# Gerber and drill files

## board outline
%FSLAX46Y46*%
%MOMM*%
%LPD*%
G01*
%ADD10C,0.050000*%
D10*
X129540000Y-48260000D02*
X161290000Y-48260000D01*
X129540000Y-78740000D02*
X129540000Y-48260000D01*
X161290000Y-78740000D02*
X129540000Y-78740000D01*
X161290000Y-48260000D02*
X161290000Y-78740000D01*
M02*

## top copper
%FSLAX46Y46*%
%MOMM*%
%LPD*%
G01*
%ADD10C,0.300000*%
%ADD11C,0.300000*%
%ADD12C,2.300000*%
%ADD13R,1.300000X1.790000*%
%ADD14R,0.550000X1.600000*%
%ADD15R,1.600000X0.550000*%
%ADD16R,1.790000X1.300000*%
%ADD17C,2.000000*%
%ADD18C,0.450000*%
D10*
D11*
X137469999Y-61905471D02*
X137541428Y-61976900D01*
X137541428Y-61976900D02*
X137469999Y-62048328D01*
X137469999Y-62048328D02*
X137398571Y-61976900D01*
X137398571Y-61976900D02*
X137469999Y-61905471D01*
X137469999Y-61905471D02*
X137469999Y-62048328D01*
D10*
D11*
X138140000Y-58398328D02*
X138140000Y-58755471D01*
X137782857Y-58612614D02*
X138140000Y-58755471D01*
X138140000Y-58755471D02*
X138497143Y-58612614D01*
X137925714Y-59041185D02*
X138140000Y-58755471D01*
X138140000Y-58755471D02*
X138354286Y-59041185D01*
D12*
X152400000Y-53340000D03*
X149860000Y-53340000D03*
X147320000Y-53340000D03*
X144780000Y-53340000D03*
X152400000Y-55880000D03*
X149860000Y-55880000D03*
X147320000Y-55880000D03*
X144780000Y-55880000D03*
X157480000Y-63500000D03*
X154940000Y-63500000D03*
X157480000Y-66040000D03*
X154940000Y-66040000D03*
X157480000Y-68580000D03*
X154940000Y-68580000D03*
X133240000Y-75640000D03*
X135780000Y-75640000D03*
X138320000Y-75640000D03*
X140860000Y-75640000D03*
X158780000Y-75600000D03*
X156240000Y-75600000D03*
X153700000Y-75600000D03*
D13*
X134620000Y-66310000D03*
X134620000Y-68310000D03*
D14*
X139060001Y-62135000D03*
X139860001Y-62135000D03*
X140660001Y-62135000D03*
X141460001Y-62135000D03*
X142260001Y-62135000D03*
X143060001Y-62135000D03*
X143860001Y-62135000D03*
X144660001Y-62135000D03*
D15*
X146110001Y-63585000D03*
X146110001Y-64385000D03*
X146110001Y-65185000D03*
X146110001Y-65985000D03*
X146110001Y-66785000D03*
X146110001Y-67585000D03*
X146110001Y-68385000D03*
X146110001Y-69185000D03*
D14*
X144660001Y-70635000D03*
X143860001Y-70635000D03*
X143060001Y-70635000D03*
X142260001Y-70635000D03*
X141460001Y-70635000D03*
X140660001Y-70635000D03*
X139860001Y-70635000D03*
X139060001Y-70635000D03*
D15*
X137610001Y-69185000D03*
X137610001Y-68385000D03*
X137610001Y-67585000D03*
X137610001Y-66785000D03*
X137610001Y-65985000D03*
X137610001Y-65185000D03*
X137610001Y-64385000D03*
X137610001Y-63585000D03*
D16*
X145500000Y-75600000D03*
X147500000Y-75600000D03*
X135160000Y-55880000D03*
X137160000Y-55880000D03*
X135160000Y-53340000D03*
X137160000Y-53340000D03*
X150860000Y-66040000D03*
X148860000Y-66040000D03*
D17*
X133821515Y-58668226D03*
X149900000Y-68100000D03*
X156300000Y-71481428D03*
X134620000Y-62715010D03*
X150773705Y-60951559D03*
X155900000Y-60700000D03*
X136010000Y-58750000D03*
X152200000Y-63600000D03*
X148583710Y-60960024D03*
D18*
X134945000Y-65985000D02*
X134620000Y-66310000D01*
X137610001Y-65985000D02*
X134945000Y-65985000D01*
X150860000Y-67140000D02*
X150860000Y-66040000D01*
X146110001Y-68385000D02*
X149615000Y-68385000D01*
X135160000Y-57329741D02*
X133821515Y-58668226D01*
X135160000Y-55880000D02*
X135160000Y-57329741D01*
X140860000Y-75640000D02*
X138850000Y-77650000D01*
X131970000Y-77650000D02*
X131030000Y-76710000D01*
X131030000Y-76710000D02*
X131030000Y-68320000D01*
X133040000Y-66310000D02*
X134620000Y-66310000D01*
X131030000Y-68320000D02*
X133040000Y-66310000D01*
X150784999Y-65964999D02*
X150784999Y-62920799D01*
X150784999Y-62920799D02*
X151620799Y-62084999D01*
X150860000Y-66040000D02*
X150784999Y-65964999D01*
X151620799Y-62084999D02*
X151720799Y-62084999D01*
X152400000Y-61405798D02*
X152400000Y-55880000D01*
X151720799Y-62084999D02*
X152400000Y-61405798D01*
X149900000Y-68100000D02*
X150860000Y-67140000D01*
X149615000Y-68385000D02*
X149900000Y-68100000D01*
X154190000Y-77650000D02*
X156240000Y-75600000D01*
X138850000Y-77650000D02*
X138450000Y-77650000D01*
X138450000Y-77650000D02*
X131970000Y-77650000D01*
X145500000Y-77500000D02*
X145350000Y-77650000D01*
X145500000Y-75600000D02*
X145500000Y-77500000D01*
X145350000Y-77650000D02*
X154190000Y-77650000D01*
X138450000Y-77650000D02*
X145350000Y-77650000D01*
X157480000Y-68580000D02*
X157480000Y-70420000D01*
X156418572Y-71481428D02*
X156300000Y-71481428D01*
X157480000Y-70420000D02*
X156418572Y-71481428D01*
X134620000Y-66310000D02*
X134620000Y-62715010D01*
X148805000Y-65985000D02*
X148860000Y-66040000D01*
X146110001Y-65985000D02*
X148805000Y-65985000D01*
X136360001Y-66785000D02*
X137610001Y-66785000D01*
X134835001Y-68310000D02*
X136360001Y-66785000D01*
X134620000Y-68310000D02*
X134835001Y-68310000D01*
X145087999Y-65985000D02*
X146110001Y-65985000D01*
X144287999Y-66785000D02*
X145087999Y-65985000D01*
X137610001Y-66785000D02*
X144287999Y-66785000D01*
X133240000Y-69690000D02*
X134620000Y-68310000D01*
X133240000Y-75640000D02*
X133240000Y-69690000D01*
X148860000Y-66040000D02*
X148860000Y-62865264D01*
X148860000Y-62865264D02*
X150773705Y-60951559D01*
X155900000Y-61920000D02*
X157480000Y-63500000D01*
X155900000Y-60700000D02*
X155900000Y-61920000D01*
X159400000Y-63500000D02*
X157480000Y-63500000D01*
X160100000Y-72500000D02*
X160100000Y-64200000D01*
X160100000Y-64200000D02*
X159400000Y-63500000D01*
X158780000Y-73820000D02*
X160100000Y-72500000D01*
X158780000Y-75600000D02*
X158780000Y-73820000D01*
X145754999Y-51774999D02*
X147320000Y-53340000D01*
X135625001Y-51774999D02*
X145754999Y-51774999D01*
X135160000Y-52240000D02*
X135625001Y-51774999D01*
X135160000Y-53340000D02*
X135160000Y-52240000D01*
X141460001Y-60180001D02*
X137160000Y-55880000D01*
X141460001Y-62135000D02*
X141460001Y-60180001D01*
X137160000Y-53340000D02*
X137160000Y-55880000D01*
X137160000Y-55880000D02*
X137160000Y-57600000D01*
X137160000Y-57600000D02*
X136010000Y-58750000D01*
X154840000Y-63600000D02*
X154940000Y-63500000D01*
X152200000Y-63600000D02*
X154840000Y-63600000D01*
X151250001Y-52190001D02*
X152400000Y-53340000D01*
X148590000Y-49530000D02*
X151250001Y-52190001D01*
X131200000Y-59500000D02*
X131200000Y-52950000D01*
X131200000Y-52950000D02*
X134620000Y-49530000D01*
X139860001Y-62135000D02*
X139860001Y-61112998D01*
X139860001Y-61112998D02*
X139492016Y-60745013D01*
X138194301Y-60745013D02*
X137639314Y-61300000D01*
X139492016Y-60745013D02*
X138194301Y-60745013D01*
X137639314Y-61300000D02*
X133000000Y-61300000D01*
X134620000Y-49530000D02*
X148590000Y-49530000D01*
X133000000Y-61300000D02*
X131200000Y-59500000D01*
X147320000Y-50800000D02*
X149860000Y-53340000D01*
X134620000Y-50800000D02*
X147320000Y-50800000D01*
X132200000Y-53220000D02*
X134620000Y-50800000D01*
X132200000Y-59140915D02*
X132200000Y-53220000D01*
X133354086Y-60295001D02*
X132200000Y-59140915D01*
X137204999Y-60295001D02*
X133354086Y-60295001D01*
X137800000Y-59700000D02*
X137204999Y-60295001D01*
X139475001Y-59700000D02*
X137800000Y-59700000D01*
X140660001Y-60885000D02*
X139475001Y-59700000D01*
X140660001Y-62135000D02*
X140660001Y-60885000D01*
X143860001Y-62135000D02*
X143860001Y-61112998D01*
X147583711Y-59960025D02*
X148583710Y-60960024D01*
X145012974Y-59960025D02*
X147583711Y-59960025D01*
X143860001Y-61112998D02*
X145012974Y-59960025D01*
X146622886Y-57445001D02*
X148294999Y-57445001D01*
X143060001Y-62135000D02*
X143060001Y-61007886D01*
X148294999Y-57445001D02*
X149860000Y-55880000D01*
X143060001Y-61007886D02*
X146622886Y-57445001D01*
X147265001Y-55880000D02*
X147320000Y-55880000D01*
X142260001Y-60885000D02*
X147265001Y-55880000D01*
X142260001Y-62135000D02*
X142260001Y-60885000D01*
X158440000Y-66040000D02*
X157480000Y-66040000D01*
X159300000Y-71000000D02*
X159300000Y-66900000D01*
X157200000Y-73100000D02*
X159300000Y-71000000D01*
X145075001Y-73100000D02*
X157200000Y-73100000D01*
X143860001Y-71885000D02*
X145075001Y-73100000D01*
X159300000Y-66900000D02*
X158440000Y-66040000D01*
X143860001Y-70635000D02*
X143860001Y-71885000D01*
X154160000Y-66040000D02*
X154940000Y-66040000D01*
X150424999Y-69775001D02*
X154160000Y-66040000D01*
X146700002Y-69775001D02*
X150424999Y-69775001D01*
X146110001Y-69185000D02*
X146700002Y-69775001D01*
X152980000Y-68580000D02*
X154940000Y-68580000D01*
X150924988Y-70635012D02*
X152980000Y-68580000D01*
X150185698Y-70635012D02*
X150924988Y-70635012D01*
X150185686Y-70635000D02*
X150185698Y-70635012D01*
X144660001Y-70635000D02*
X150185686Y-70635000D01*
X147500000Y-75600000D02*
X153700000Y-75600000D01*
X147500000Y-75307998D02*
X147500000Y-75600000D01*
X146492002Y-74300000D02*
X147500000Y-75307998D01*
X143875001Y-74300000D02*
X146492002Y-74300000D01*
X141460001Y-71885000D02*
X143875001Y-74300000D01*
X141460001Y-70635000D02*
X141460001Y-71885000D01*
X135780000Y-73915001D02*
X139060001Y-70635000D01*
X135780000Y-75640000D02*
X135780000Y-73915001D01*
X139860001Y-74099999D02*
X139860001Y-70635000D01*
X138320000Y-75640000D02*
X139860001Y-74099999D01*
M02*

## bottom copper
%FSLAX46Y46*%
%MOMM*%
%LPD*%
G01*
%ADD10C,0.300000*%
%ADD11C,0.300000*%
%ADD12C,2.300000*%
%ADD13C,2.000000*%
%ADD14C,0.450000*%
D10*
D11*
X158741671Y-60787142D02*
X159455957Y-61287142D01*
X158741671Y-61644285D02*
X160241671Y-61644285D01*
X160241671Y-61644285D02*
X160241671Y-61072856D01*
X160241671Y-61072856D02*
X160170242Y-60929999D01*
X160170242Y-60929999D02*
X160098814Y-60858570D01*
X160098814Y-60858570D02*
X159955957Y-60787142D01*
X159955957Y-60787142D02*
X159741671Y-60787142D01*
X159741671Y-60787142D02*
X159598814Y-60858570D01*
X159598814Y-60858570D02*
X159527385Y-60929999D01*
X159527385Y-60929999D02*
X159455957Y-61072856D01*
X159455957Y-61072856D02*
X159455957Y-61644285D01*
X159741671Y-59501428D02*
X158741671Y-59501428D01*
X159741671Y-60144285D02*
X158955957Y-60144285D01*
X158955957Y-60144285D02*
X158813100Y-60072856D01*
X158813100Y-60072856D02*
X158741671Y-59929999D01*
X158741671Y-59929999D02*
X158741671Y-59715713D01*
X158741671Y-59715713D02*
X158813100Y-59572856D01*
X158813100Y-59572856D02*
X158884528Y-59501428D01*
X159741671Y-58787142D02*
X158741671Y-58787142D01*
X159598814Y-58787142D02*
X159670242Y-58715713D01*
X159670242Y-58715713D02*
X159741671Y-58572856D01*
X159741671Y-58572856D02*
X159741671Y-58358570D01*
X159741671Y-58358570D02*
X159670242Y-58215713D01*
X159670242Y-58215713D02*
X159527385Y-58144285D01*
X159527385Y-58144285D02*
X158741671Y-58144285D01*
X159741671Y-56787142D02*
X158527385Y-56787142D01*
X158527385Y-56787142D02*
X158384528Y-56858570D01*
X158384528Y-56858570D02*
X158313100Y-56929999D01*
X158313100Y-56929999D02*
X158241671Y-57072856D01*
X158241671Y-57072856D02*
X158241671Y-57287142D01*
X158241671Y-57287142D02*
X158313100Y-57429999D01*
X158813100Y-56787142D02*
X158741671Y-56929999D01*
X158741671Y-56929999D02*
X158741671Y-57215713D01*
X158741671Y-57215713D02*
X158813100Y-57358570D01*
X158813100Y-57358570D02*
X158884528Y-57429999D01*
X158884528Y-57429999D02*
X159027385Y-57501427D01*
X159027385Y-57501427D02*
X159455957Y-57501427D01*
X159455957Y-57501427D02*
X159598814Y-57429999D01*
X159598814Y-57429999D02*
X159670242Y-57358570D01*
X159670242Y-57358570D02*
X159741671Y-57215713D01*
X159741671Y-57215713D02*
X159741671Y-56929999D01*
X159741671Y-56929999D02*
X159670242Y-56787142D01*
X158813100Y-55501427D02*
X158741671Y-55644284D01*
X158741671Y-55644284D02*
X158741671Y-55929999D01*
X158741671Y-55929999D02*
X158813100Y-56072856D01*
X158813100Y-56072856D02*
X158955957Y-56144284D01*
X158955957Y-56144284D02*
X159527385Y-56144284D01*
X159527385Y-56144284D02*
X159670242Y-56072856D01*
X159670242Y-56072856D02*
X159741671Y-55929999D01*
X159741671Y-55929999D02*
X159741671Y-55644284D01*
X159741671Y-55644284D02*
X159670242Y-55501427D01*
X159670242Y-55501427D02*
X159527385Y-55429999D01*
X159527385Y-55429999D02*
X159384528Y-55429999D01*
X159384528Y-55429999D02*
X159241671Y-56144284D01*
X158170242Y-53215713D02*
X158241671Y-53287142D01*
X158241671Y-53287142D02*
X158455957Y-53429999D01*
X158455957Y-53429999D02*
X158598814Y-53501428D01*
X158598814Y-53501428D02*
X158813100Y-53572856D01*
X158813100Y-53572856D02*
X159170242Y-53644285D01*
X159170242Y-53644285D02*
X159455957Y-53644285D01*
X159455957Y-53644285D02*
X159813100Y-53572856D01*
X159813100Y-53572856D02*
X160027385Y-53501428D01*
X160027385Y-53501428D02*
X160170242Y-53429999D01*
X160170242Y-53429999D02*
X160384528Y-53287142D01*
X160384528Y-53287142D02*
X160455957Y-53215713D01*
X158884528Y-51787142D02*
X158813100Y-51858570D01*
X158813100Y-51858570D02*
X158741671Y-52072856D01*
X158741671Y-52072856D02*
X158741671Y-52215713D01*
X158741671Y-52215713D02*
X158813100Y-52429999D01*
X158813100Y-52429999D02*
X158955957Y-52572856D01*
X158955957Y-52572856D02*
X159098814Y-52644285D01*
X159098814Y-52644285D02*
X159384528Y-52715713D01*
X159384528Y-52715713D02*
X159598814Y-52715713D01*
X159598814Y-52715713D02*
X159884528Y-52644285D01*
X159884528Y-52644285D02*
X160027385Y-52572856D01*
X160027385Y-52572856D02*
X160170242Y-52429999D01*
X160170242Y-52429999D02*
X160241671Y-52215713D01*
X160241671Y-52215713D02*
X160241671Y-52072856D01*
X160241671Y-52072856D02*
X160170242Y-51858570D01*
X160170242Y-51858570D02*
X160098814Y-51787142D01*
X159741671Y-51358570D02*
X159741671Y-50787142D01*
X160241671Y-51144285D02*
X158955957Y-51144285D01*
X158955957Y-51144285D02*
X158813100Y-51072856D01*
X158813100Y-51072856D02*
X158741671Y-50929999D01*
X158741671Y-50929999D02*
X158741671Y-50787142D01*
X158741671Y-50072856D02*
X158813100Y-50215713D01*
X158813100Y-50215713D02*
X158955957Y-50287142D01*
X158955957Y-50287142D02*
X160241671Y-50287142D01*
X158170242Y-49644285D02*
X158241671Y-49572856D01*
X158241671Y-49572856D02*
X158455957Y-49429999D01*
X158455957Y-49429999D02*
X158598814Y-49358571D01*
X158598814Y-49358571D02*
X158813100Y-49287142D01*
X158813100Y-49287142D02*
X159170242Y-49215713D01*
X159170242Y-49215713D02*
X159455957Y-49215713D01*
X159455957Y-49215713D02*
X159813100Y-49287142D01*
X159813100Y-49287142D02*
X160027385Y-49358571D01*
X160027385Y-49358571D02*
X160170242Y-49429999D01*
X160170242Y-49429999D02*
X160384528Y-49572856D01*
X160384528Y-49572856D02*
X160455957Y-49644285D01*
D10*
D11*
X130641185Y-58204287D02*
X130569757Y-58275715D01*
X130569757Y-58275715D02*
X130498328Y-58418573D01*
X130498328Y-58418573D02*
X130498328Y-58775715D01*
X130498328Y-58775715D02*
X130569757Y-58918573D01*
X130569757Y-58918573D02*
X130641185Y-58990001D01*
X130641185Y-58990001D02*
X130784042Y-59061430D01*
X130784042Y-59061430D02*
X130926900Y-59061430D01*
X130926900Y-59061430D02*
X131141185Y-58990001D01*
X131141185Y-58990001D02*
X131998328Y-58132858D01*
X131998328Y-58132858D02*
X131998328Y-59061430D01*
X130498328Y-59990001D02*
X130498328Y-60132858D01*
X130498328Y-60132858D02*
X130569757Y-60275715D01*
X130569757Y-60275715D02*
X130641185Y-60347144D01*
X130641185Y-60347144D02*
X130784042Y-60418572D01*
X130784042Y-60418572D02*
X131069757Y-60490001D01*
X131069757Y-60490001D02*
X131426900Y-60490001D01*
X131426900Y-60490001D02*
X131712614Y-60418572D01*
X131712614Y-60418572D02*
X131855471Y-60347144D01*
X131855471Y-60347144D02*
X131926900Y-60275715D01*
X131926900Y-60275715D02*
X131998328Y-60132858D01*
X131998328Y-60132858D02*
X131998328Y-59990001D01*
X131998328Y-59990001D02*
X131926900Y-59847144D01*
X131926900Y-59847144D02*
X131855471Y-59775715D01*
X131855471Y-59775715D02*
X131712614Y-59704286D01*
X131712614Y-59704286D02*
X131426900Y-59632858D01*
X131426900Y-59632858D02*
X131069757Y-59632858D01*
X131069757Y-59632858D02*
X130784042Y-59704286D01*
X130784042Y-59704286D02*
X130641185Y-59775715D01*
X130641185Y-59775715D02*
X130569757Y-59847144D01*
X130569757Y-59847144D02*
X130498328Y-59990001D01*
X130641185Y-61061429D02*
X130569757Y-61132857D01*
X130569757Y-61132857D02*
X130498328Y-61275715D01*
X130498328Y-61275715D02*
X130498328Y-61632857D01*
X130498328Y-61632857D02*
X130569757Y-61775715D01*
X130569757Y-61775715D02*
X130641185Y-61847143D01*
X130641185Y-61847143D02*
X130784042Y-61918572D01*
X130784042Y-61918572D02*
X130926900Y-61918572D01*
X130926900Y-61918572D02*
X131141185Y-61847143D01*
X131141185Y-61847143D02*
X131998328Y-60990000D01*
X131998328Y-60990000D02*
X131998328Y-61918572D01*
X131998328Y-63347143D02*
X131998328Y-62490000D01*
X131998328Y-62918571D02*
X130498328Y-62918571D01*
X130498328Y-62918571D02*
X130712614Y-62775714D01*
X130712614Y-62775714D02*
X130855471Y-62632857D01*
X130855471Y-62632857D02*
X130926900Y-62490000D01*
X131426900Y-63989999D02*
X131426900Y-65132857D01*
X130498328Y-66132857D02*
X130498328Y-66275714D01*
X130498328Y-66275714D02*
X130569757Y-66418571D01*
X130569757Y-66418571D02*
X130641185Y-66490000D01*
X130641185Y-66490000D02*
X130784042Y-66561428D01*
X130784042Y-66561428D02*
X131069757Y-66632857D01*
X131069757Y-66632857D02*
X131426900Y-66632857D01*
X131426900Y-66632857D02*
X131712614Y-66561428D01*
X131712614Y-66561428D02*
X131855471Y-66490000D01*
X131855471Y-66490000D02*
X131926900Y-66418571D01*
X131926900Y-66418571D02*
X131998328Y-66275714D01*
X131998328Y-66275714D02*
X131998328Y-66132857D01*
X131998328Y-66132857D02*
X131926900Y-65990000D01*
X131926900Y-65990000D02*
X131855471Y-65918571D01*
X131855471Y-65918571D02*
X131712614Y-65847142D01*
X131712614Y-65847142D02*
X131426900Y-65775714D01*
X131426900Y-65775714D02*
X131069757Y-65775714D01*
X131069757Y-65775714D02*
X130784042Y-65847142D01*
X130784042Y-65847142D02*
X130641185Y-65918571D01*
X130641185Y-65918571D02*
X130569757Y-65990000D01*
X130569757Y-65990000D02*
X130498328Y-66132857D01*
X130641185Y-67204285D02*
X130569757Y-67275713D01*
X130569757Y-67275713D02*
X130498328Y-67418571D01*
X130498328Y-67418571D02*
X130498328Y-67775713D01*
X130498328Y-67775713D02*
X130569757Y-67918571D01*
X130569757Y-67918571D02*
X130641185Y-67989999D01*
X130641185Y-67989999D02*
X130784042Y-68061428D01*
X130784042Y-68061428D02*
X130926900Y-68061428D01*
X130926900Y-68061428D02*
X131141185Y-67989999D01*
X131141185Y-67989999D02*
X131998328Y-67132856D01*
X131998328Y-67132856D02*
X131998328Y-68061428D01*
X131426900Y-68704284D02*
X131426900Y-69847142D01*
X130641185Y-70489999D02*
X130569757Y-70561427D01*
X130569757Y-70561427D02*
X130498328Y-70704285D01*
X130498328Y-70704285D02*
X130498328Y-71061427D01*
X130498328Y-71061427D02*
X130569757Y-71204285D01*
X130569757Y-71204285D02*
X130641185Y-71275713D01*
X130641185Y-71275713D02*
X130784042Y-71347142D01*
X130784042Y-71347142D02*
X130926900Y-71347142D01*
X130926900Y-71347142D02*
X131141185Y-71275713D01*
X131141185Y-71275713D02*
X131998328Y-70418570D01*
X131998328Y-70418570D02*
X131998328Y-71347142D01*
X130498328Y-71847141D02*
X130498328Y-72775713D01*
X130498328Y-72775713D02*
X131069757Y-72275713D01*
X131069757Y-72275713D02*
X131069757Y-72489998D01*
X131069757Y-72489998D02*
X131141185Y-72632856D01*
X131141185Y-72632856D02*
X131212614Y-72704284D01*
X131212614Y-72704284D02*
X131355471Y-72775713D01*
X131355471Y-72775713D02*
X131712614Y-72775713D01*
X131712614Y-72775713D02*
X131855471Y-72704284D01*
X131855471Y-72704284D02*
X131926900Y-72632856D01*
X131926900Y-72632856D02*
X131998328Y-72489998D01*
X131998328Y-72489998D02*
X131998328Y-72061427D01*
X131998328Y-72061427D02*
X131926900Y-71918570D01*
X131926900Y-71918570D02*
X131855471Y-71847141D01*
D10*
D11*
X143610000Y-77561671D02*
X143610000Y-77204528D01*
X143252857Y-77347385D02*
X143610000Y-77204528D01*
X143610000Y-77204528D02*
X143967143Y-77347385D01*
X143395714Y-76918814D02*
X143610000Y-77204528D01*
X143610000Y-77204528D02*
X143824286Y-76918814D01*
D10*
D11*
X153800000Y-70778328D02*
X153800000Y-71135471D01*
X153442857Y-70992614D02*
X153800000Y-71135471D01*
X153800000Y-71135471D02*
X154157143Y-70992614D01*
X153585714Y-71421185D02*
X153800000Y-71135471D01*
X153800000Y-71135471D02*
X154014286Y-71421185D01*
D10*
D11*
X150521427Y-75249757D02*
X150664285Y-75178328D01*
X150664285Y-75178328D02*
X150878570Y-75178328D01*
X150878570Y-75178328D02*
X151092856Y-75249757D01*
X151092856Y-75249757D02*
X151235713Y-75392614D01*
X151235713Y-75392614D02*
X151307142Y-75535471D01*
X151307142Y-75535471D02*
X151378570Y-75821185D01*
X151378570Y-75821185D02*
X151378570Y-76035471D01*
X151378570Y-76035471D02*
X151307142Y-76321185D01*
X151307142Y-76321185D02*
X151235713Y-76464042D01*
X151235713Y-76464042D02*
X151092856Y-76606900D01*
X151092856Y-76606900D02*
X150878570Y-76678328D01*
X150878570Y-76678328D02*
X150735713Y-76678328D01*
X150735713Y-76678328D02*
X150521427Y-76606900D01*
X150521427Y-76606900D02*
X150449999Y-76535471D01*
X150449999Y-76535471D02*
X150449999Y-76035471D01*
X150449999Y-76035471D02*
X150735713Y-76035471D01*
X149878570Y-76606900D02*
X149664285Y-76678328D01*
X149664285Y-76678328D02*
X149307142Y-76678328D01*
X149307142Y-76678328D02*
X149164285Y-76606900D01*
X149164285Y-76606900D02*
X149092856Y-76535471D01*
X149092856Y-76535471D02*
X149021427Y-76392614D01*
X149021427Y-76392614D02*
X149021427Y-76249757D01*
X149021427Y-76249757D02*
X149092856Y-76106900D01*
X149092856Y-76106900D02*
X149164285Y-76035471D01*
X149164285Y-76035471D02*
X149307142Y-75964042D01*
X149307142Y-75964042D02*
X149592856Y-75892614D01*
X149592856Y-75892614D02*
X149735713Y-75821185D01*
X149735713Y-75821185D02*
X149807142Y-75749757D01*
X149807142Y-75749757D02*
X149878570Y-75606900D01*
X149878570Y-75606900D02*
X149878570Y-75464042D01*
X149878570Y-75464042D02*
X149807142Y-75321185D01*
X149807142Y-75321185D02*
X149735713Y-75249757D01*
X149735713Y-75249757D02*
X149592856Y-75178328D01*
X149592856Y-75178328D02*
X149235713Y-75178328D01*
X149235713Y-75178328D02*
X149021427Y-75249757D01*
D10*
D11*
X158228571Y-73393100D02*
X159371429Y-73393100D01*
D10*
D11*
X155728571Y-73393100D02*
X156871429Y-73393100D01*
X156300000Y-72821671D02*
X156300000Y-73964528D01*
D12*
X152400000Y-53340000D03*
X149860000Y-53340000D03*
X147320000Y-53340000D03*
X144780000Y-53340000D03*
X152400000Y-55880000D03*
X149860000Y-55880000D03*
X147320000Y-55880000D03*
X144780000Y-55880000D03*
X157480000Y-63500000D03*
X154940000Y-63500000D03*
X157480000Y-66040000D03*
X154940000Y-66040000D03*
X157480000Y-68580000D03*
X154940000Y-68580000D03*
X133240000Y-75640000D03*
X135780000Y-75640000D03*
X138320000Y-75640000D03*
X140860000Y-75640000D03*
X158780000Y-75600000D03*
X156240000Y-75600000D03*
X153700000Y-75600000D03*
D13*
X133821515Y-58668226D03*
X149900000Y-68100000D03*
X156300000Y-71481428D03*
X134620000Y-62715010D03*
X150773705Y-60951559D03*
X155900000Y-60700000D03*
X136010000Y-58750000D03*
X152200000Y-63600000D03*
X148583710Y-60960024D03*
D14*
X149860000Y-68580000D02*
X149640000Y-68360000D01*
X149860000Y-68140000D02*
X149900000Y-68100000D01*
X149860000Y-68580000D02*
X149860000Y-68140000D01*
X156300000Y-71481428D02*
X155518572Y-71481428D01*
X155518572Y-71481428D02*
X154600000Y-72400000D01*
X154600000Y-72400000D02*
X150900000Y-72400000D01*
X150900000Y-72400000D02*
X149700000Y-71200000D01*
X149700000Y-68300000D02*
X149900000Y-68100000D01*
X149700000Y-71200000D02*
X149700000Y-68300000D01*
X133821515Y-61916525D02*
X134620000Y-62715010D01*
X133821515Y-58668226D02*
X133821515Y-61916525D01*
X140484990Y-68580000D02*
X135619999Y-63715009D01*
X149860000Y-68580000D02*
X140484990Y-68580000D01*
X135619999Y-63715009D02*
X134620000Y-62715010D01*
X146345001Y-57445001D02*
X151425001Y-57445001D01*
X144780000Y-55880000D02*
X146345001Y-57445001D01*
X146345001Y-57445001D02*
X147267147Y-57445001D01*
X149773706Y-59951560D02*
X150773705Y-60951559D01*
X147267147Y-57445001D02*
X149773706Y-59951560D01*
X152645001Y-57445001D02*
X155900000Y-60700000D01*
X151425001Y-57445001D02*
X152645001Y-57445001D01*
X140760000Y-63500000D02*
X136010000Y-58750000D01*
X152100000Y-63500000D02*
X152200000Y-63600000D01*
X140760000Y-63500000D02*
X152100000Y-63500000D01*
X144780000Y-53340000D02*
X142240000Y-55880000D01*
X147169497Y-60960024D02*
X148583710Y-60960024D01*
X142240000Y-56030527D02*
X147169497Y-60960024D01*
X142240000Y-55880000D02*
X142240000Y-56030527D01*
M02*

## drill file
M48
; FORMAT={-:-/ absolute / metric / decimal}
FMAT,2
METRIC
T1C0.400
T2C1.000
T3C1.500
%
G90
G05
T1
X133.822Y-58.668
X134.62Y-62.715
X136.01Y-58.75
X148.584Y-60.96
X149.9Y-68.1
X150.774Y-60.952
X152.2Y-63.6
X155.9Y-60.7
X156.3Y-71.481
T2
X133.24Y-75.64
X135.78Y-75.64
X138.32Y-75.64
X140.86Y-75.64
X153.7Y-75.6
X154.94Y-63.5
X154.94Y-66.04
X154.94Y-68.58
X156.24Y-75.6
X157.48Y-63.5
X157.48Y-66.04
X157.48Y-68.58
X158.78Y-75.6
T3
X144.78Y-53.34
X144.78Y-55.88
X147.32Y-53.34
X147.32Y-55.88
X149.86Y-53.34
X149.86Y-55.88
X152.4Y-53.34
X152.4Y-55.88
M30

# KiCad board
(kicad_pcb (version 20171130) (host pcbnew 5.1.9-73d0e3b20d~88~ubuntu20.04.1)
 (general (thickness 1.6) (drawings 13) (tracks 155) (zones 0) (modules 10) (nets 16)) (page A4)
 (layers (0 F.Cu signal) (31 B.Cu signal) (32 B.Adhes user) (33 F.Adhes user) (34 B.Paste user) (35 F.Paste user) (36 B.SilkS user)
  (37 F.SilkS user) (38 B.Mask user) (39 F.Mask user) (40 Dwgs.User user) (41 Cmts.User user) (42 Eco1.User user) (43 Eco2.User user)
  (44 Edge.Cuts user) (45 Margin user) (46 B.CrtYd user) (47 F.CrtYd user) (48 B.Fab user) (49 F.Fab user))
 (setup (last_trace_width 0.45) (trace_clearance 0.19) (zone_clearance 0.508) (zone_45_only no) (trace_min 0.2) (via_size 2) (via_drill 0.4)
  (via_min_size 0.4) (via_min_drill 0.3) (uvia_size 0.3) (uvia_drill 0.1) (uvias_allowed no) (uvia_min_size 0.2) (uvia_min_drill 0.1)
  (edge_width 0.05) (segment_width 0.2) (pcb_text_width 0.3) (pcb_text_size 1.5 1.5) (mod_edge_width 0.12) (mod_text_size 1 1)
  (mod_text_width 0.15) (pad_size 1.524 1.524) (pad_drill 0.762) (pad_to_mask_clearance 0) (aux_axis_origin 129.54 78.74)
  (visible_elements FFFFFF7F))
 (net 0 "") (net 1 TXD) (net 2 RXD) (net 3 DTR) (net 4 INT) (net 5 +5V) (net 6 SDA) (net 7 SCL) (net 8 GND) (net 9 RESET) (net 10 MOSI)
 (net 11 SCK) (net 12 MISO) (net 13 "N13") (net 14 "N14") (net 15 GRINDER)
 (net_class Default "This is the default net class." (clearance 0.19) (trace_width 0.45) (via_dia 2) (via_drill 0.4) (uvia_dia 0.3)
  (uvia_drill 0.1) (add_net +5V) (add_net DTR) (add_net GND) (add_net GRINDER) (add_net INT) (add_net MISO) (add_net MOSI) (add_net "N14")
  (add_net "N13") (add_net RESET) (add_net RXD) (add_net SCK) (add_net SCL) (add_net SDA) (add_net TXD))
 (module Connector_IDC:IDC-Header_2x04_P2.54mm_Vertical (layer F.Cu) (at 144.78 55.88 90)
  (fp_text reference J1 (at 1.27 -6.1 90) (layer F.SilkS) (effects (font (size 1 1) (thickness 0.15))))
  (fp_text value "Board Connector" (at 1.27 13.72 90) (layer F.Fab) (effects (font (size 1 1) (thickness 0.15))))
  (pad 8 thru_hole circle (at 2.54 7.62 90) (size 2.3 2.3) (drill 1.5) (layers *.Cu *.Mask) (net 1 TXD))
  (pad 6 thru_hole circle (at 2.54 5.08 90) (size 2.3 2.3) (drill 1.5) (layers *.Cu *.Mask) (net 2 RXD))
  (pad 4 thru_hole circle (at 2.54 2.54 90) (size 2.3 2.3) (drill 1.5) (layers *.Cu *.Mask) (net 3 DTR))
  (pad 2 thru_hole circle (at 2.54 0 90) (size 2.3 2.3) (drill 1.5) (layers *.Cu *.Mask) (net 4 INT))
  (pad 7 thru_hole circle (at 0 7.62 90) (size 2.3 2.3) (drill 1.5) (layers *.Cu *.Mask) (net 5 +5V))
  (pad 5 thru_hole circle (at 0 5.08 90) (size 2.3 2.3) (drill 1.5) (layers *.Cu *.Mask) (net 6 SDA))
  (pad 3 thru_hole circle (at 0 2.54 90) (size 2.3 2.3) (drill 1.5) (layers *.Cu *.Mask) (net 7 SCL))
  (pad 1 thru_hole circle (at 0 0 90) (size 2.3 2.3) (drill 1.5) (layers *.Cu *.Mask) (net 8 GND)))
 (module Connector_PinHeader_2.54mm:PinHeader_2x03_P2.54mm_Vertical (layer B.Cu) (at 154.94 68.58)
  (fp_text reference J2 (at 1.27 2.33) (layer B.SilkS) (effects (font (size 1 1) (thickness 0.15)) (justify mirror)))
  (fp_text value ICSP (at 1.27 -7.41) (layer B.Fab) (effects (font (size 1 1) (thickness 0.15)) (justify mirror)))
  (pad 6 thru_hole circle (at 2.54 -5.08) (size 2.3 2.3) (drill 1) (layers *.Cu *.Mask) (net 8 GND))
  (pad 5 thru_hole circle (at 0 -5.08) (size 2.3 2.3) (drill 1) (layers *.Cu *.Mask) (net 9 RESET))
  (pad 4 thru_hole circle (at 2.54 -2.54) (size 2.3 2.3) (drill 1) (layers *.Cu *.Mask) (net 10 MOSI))
  (pad 3 thru_hole circle (at 0 -2.54) (size 2.3 2.3) (drill 1) (layers *.Cu *.Mask) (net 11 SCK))
  (pad 2 thru_hole circle (at 2.54 0) (size 2.3 2.3) (drill 1) (layers *.Cu *.Mask) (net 5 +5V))
  (pad 1 thru_hole circle (at 0 0) (size 2.3 2.3) (drill 1) (layers *.Cu *.Mask) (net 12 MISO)))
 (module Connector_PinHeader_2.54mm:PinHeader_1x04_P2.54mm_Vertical (layer B.Cu) (at 140.86 75.64 90)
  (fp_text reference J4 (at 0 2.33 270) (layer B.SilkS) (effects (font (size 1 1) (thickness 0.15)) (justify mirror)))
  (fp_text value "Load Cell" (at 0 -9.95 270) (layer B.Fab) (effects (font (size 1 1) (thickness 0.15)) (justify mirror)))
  (pad 4 thru_hole circle (at 0 -7.62 90) (size 2.3 2.3) (drill 1) (layers *.Cu *.Mask) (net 8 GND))
  (pad 3 thru_hole circle (at 0 -5.08 90) (size 2.3 2.3) (drill 1) (layers *.Cu *.Mask) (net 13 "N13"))
  (pad 2 thru_hole circle (at 0 -2.54 90) (size 2.3 2.3) (drill 1) (layers *.Cu *.Mask) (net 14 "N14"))
  (pad 1 thru_hole circle (at 0 0 90) (size 2.3 2.3) (drill 1) (layers *.Cu *.Mask) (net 5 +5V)))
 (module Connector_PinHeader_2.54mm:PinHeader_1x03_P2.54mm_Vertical (layer B.Cu) (at 153.7 75.6 270)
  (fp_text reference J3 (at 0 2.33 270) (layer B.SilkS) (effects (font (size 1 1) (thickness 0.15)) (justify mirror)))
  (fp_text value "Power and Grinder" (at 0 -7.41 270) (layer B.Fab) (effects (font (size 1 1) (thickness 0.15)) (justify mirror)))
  (pad 3 thru_hole circle (at 0 -5.08 270) (size 2.3 2.3) (drill 1) (layers *.Cu *.Mask) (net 8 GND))
  (pad 2 thru_hole circle (at 0 -2.54 270) (size 2.3 2.3) (drill 1) (layers *.Cu *.Mask) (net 5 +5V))
  (pad 1 thru_hole circle (at 0 0 270) (size 2.3 2.3) (drill 1) (layers *.Cu *.Mask) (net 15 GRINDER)))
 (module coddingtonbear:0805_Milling (layer F.Cu) (at 134.62 67.31 270)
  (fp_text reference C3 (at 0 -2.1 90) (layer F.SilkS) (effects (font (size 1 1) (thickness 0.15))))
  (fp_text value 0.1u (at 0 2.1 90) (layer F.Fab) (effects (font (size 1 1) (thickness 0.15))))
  (pad 1 smd rect (at -1 0 270) (size 1.79 1.3) (layers F.Cu F.Paste F.Mask) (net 5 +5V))
  (pad 2 smd rect (at 1 0 270) (size 1.79 1.3) (layers F.Cu F.Paste F.Mask) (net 8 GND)))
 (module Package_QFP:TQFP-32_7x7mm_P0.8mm (layer F.Cu) (at 141.860001 66.385)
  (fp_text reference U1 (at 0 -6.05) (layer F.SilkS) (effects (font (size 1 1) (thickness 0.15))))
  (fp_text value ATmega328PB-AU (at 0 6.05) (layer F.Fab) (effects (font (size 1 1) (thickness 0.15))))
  (pad 32 smd rect (at -2.8 -4.25 90) (size 1.6 0.55) (layers F.Cu F.Paste F.Mask))
  (pad 31 smd rect (at -2 -4.25 90) (size 1.6 0.55) (layers F.Cu F.Paste F.Mask) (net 1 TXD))
  (pad 30 smd rect (at -1.2 -4.25 90) (size 1.6 0.55) (layers F.Cu F.Paste F.Mask) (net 2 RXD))
  (pad 29 smd rect (at -0.4 -4.25 90) (size 1.6 0.55) (layers F.Cu F.Paste F.Mask) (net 9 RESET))
  (pad 28 smd rect (at 0.4 -4.25 90) (size 1.6 0.55) (layers F.Cu F.Paste F.Mask) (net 7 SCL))
  (pad 27 smd rect (at 1.2 -4.25 90) (size 1.6 0.55) (layers F.Cu F.Paste F.Mask) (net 6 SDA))
  (pad 26 smd rect (at 2 -4.25 90) (size 1.6 0.55) (layers F.Cu F.Paste F.Mask) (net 4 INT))
  (pad 25 smd rect (at 2.8 -4.25 90) (size 1.6 0.55) (layers F.Cu F.Paste F.Mask))
  (pad 24 smd rect (at 4.25 -2.8) (size 1.6 0.55) (layers F.Cu F.Paste F.Mask))
  (pad 23 smd rect (at 4.25 -2) (size 1.6 0.55) (layers F.Cu F.Paste F.Mask))
  (pad 22 smd rect (at 4.25 -1.2) (size 1.6 0.55) (layers F.Cu F.Paste F.Mask))
  (pad 21 smd rect (at 4.25 -0.4) (size 1.6 0.55) (layers F.Cu F.Paste F.Mask) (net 8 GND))
  (pad 20 smd rect (at 4.25 0.4) (size 1.6 0.55) (layers F.Cu F.Paste F.Mask))
  (pad 19 smd rect (at 4.25 1.2) (size 1.6 0.55) (layers F.Cu F.Paste F.Mask))
  (pad 18 smd rect (at 4.25 2) (size 1.6 0.55) (layers F.Cu F.Paste F.Mask) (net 5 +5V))
  (pad 17 smd rect (at 4.25 2.8) (size 1.6 0.55) (layers F.Cu F.Paste F.Mask) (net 11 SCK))
  (pad 16 smd rect (at 2.8 4.25 90) (size 1.6 0.55) (layers F.Cu F.Paste F.Mask) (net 12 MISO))
  (pad 15 smd rect (at 2 4.25 90) (size 1.6 0.55) (layers F.Cu F.Paste F.Mask) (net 10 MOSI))
  (pad 14 smd rect (at 1.2 4.25 90) (size 1.6 0.55) (layers F.Cu F.Paste F.Mask))
  (pad 13 smd rect (at 0.4 4.25 90) (size 1.6 0.55) (layers F.Cu F.Paste F.Mask))
  (pad 12 smd rect (at -0.4 4.25 90) (size 1.6 0.55) (layers F.Cu F.Paste F.Mask) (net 15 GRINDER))
  (pad 11 smd rect (at -1.2 4.25 90) (size 1.6 0.55) (layers F.Cu F.Paste F.Mask))
  (pad 10 smd rect (at -2 4.25 90) (size 1.6 0.55) (layers F.Cu F.Paste F.Mask) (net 14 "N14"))
  (pad 9 smd rect (at -2.8 4.25 90) (size 1.6 0.55) (layers F.Cu F.Paste F.Mask) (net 13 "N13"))
  (pad 8 smd rect (at -4.25 2.8) (size 1.6 0.55) (layers F.Cu F.Paste F.Mask))
  (pad 7 smd rect (at -4.25 2) (size 1.6 0.55) (layers F.Cu F.Paste F.Mask))
  (pad 6 smd rect (at -4.25 1.2) (size 1.6 0.55) (layers F.Cu F.Paste F.Mask))
  (pad 5 smd rect (at -4.25 0.4) (size 1.6 0.55) (layers F.Cu F.Paste F.Mask) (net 8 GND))
  (pad 4 smd rect (at -4.25 -0.4) (size 1.6 0.55) (layers F.Cu F.Paste F.Mask) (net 5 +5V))
  (pad 3 smd rect (at -4.25 -1.2) (size 1.6 0.55) (layers F.Cu F.Paste F.Mask))
  (pad 2 smd rect (at -4.25 -2) (size 1.6 0.55) (layers F.Cu F.Paste F.Mask))
  (pad 1 smd rect (at -4.25 -2.8) (size 1.6 0.55) (layers F.Cu F.Paste F.Mask)))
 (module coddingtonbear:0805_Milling (layer F.Cu) (at 146.5 75.6)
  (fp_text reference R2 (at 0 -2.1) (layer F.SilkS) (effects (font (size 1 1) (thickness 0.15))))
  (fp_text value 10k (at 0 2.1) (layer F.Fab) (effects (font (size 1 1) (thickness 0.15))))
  (pad 1 smd rect (at -1 0) (size 1.79 1.3) (layers F.Cu F.Paste F.Mask) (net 5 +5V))
  (pad 2 smd rect (at 1 0) (size 1.79 1.3) (layers F.Cu F.Paste F.Mask) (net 15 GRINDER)))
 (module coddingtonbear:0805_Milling (layer F.Cu) (at 136.16 55.88)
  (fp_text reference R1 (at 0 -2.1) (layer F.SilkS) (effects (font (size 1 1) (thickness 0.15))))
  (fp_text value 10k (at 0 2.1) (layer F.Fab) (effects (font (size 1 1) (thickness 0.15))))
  (pad 1 smd rect (at -1 0) (size 1.79 1.3) (layers F.Cu F.Paste F.Mask) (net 5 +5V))
  (pad 2 smd rect (at 1 0) (size 1.79 1.3) (layers F.Cu F.Paste F.Mask) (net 9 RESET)))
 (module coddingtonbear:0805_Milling (layer F.Cu) (at 136.16 53.34)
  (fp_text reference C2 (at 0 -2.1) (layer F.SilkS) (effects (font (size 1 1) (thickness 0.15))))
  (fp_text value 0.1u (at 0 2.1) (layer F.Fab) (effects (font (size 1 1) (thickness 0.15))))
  (pad 1 smd rect (at -1 0) (size 1.79 1.3) (layers F.Cu F.Paste F.Mask) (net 3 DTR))
  (pad 2 smd rect (at 1 0) (size 1.79 1.3) (layers F.Cu F.Paste F.Mask) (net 9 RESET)))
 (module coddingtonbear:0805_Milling (layer F.Cu) (at 149.86 66.04 180)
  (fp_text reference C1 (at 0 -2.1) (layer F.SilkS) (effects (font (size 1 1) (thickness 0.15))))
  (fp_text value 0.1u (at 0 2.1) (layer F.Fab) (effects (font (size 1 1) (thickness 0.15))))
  (pad 1 smd rect (at -1 0 180) (size 1.79 1.3) (layers F.Cu F.Paste F.Mask) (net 5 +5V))
  (pad 2 smd rect (at 1 0 180) (size 1.79 1.3) (layers F.Cu F.Paste F.Mask) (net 8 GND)))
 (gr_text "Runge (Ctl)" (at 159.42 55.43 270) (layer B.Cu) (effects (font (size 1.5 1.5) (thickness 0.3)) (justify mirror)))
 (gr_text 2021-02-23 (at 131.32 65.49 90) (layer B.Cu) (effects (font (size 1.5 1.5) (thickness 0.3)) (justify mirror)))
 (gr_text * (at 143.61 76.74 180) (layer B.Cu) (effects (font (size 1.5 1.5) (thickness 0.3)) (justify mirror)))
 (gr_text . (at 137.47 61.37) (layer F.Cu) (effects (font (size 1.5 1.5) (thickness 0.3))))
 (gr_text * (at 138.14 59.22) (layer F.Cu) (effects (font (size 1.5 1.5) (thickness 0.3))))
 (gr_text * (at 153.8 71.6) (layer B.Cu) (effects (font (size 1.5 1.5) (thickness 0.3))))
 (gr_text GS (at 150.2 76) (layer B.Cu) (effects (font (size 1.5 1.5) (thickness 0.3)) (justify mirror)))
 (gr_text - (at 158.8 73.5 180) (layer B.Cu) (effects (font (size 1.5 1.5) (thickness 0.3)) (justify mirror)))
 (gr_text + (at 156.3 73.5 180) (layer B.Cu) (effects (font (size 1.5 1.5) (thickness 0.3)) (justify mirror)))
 (gr_line (start 129.54 48.26) (end 161.29 48.26) (layer Edge.Cuts) (width 0.05))
 (gr_line (start 129.54 78.74) (end 129.54 48.26) (layer Edge.Cuts) (width 0.05))
 (gr_line (start 161.29 78.74) (end 129.54 78.74) (layer Edge.Cuts) (width 0.05))
 (gr_line (start 161.29 48.26) (end 161.29 78.74) (layer Edge.Cuts) (width 0.05))
 (segment (start 134.945 65.985) (end 134.62 66.31) (width 0.45) (layer F.Cu) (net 5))
 (segment (start 137.610001 65.985) (end 134.945 65.985) (width 0.45) (layer F.Cu) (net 5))
 (segment (start 150.86 67.14) (end 150.86 66.04) (width 0.45) (layer F.Cu) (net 5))
 (segment (start 146.110001 68.385) (end 149.615 68.385) (width 0.45) (layer F.Cu) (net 5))
 (segment (start 149.86 68.58) (end 149.64 68.36) (width 0.45) (layer B.Cu) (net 5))
 (via (at 133.821515 58.668226) (size 2) (drill 0.4) (layers F.Cu B.Cu) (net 5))
 (segment (start 135.16 57.329741) (end 133.821515 58.668226) (width 0.45) (layer F.Cu) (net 5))
 (segment (start 135.16 55.88) (end 135.16 57.329741) (width 0.45) (layer F.Cu) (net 5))
 (segment (start 140.86 75.64) (end 138.85 77.65) (width 0.45) (layer F.Cu) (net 5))
 (segment (start 131.97 77.65) (end 131.03 76.71) (width 0.45) (layer F.Cu) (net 5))
 (segment (start 131.03 76.71) (end 131.03 68.32) (width 0.45) (layer F.Cu) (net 5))
 (segment (start 133.04 66.31) (end 134.62 66.31) (width 0.45) (layer F.Cu) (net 5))
 (segment (start 131.03 68.32) (end 133.04 66.31) (width 0.45) (layer F.Cu) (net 5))
 (segment (start 150.784999 65.964999) (end 150.784999 62.920799) (width 0.45) (layer F.Cu) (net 5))
 (segment (start 150.784999 62.920799) (end 151.620799 62.084999) (width 0.45) (layer F.Cu) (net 5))
 (segment (start 150.86 66.04) (end 150.784999 65.964999) (width 0.45) (layer F.Cu) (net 5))
 (segment (start 151.620799 62.084999) (end 151.720799 62.084999) (width 0.45) (layer F.Cu) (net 5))
 (segment (start 152.4 61.405798) (end 152.4 55.88) (width 0.45) (layer F.Cu) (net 5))
 (segment (start 151.720799 62.084999) (end 152.4 61.405798) (width 0.45) (layer F.Cu) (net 5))
 (segment (start 149.86 68.14) (end 149.9 68.1) (width 0.45) (layer B.Cu) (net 5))
 (segment (start 149.86 68.58) (end 149.86 68.14) (width 0.45) (layer B.Cu) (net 5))
 (segment (start 149.9 68.1) (end 150.86 67.14) (width 0.45) (layer F.Cu) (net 5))
 (via (at 149.9 68.1) (size 2) (drill 0.4) (layers F.Cu B.Cu) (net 5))
 (segment (start 149.615 68.385) (end 149.9 68.1) (width 0.45) (layer F.Cu) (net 5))
 (segment (start 154.19 77.65) (end 156.24 75.6) (width 0.45) (layer F.Cu) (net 5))
 (segment (start 138.85 77.65) (end 138.45 77.65) (width 0.45) (layer F.Cu) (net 5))
 (segment (start 138.45 77.65) (end 131.97 77.65) (width 0.45) (layer F.Cu) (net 5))
 (segment (start 145.5 77.5) (end 145.35 77.65) (width 0.45) (layer F.Cu) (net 5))
 (segment (start 145.5 75.6) (end 145.5 77.5) (width 0.45) (layer F.Cu) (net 5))
 (segment (start 145.35 77.65) (end 154.19 77.65) (width 0.45) (layer F.Cu) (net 5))
 (segment (start 138.45 77.65) (end 145.35 77.65) (width 0.45) (layer F.Cu) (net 5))
 (segment (start 157.48 68.58) (end 157.48 70.42) (width 0.45) (layer F.Cu) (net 5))
 (via (at 156.3 71.481428) (size 2) (drill 0.4) (layers F.Cu B.Cu) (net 5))
 (segment (start 156.418572 71.481428) (end 156.3 71.481428) (width 0.45) (layer F.Cu) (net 5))
 (segment (start 157.48 70.42) (end 156.418572 71.481428) (width 0.45) (layer F.Cu) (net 5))
 (segment (start 156.3 71.481428) (end 155.518572 71.481428) (width 0.45) (layer B.Cu) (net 5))
 (segment (start 155.518572 71.481428) (end 154.6 72.4) (width 0.45) (layer B.Cu) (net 5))
 (segment (start 154.6 72.4) (end 150.9 72.4) (width 0.45) (layer B.Cu) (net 5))
 (segment (start 150.9 72.4) (end 149.7 71.2) (width 0.45) (layer B.Cu) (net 5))
 (segment (start 149.7 68.3) (end 149.9 68.1) (width 0.45) (layer B.Cu) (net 5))
 (segment (start 149.7 71.2) (end 149.7 68.3) (width 0.45) (layer B.Cu) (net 5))
 (segment (start 133.821515 61.916525) (end 134.62 62.71501) (width 0.45) (layer B.Cu) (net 5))
 (segment (start 133.821515 58.668226) (end 133.821515 61.916525) (width 0.45) (layer B.Cu) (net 5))
 (segment (start 140.48499 68.58) (end 135.619999 63.715009) (width 0.45) (layer B.Cu) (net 5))
 (via (at 134.62 62.71501) (size 2) (drill 0.4) (layers F.Cu B.Cu) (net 5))
 (segment (start 134.62 66.31) (end 134.62 62.71501) (width 0.45) (layer F.Cu) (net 5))
 (segment (start 149.86 68.58) (end 140.48499 68.58) (width 0.45) (layer B.Cu) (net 5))
 (segment (start 135.619999 63.715009) (end 134.62 62.71501) (width 0.45) (layer B.Cu) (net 5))
 (segment (start 146.345001 57.445001) (end 151.425001 57.445001) (width 0.45) (layer B.Cu) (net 8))
 (segment (start 144.78 55.88) (end 146.345001 57.445001) (width 0.45) (layer B.Cu) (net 8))
 (segment (start 148.805 65.985) (end 148.86 66.04) (width 0.45) (layer F.Cu) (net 8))
 (segment (start 146.110001 65.985) (end 148.805 65.985) (width 0.45) (layer F.Cu) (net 8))
 (segment (start 136.360001 66.785) (end 137.610001 66.785) (width 0.45) (layer F.Cu) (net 8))
 (segment (start 134.835001 68.31) (end 136.360001 66.785) (width 0.45) (layer F.Cu) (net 8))
 (segment (start 134.62 68.31) (end 134.835001 68.31) (width 0.45) (layer F.Cu) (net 8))
 (segment (start 145.087999 65.985) (end 146.110001 65.985) (width 0.45) (layer F.Cu) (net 8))
 (segment (start 144.287999 66.785) (end 145.087999 65.985) (width 0.45) (layer F.Cu) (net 8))
 (segment (start 137.610001 66.785) (end 144.287999 66.785) (width 0.45) (layer F.Cu) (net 8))
 (segment (start 133.24 69.69) (end 134.62 68.31) (width 0.45) (layer F.Cu) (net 8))
 (segment (start 133.24 75.64) (end 133.24 69.69) (width 0.45) (layer F.Cu) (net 8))
 (segment (start 146.345001 57.445001) (end 147.267147 57.445001) (width 0.45) (layer B.Cu) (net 8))
 (segment (start 149.773706 59.95156) (end 150.773705 60.951559) (width 0.45) (layer B.Cu) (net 8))
 (segment (start 147.267147 57.445001) (end 149.773706 59.95156) (width 0.45) (layer B.Cu) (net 8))
 (via (at 150.773705 60.951559) (size 2) (drill 0.4) (layers F.Cu B.Cu) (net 8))
 (segment (start 148.86 66.04) (end 148.86 62.865264) (width 0.45) (layer F.Cu) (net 8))
 (segment (start 148.86 62.865264) (end 150.773705 60.951559) (width 0.45) (layer F.Cu) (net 8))
 (segment (start 152.645001 57.445001) (end 155.9 60.7) (width 0.45) (layer B.Cu) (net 8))
 (via (at 155.9 60.7) (size 2) (drill 0.4) (layers F.Cu B.Cu) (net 8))
 (segment (start 151.425001 57.445001) (end 152.645001 57.445001) (width 0.45) (layer B.Cu) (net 8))
 (segment (start 155.9 61.92) (end 157.48 63.5) (width 0.45) (layer F.Cu) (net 8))
 (segment (start 155.9 60.7) (end 155.9 61.92) (width 0.45) (layer F.Cu) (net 8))
 (segment (start 159.4 63.5) (end 157.48 63.5) (width 0.45) (layer F.Cu) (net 8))
 (segment (start 160.1 72.5) (end 160.1 64.2) (width 0.45) (layer F.Cu) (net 8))
 (segment (start 160.1 64.2) (end 159.4 63.5) (width 0.45) (layer F.Cu) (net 8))
 (segment (start 158.78 73.82) (end 160.1 72.5) (width 0.45) (layer F.Cu) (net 8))
 (segment (start 158.78 75.6) (end 158.78 73.82) (width 0.45) (layer F.Cu) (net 8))
 (segment (start 145.754999 51.774999) (end 147.32 53.34) (width 0.45) (layer F.Cu) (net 3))
 (segment (start 135.625001 51.774999) (end 145.754999 51.774999) (width 0.45) (layer F.Cu) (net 3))
 (segment (start 135.16 52.24) (end 135.625001 51.774999) (width 0.45) (layer F.Cu) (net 3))
 (segment (start 135.16 53.34) (end 135.16 52.24) (width 0.45) (layer F.Cu) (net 3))
 (segment (start 141.460001 60.180001) (end 137.16 55.88) (width 0.45) (layer F.Cu) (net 9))
 (segment (start 141.460001 62.135) (end 141.460001 60.180001) (width 0.45) (layer F.Cu) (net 9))
 (segment (start 137.16 53.34) (end 137.16 55.88) (width 0.45) (layer F.Cu) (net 9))
 (via (at 136.01 58.75) (size 2) (drill 0.4) (layers F.Cu B.Cu) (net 9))
 (segment (start 137.16 55.88) (end 137.16 57.6) (width 0.45) (layer F.Cu) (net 9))
 (segment (start 137.16 57.6) (end 136.01 58.75) (width 0.45) (layer F.Cu) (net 9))
 (segment (start 140.76 63.5) (end 136.01 58.75) (width 0.45) (layer B.Cu) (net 9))
 (via (at 152.2 63.6) (size 2) (drill 0.4) (layers F.Cu B.Cu) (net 9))
 (segment (start 152.1 63.5) (end 152.2 63.6) (width 0.45) (layer B.Cu) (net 9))
 (segment (start 140.76 63.5) (end 152.1 63.5) (width 0.45) (layer B.Cu) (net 9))
 (segment (start 154.84 63.6) (end 154.94 63.5) (width 0.45) (layer F.Cu) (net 9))
 (segment (start 152.2 63.6) (end 154.84 63.6) (width 0.45) (layer F.Cu) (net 9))
 (segment (start 151.250001 52.190001) (end 152.4 53.34) (width 0.45) (layer F.Cu) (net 1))
 (segment (start 148.59 49.53) (end 151.250001 52.190001) (width 0.45) (layer F.Cu) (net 1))
 (segment (start 131.2 59.5) (end 131.2 52.95) (width 0.45) (layer F.Cu) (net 1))
 (segment (start 131.2 52.95) (end 134.62 49.53) (width 0.45) (layer F.Cu) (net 1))
 (segment (start 139.860001 62.135) (end 139.860001 61.112998) (width 0.45) (layer F.Cu) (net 1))
 (segment (start 139.860001 61.112998) (end 139.492016 60.745013) (width 0.45) (layer F.Cu) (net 1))
 (segment (start 138.194301 60.745013) (end 137.639314 61.3) (width 0.45) (layer F.Cu) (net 1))
 (segment (start 139.492016 60.745013) (end 138.194301 60.745013) (width 0.45) (layer F.Cu) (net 1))
 (segment (start 137.639314 61.3) (end 133 61.3) (width 0.45) (layer F.Cu) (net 1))
 (segment (start 134.62 49.53) (end 148.59 49.53) (width 0.45) (layer F.Cu) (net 1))
 (segment (start 133 61.3) (end 131.2 59.5) (width 0.45) (layer F.Cu) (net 1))
 (segment (start 147.32 50.8) (end 149.86 53.34) (width 0.45) (layer F.Cu) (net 2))
 (segment (start 134.62 50.8) (end 147.32 50.8) (width 0.45) (layer F.Cu) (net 2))
 (segment (start 132.2 53.22) (end 134.62 50.8) (width 0.45) (layer F.Cu) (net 2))
 (segment (start 132.2 59.140915) (end 132.2 53.22) (width 0.45) (layer F.Cu) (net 2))
 (segment (start 133.354086 60.295001) (end 132.2 59.140915) (width 0.45) (layer F.Cu) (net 2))
 (segment (start 137.204999 60.295001) (end 133.354086 60.295001) (width 0.45) (layer F.Cu) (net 2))
 (segment (start 137.8 59.7) (end 137.204999 60.295001) (width 0.45) (layer F.Cu) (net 2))
 (segment (start 139.475001 59.7) (end 137.8 59.7) (width 0.45) (layer F.Cu) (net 2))
 (segment (start 140.660001 60.885) (end 139.475001 59.7) (width 0.45) (layer F.Cu) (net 2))
 (segment (start 140.660001 62.135) (end 140.660001 60.885) (width 0.45) (layer F.Cu) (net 2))
 (segment (start 143.860001 62.135) (end 143.860001 61.112998) (width 0.45) (layer F.Cu) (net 4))
 (segment (start 144.78 53.34) (end 142.24 55.88) (width 0.45) (layer B.Cu) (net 4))
 (via (at 148.58371 60.960024) (size 2) (drill 0.4) (layers F.Cu B.Cu) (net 4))
 (segment (start 147.169497 60.960024) (end 148.58371 60.960024) (width 0.45) (layer B.Cu) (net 4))
 (segment (start 147.583711 59.960025) (end 148.58371 60.960024) (width 0.45) (layer F.Cu) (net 4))
 (segment (start 142.24 56.030527) (end 147.169497 60.960024) (width 0.45) (layer B.Cu) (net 4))
 (segment (start 145.012974 59.960025) (end 147.583711 59.960025) (width 0.45) (layer F.Cu) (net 4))
 (segment (start 142.24 55.88) (end 142.24 56.030527) (width 0.45) (layer B.Cu) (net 4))
 (segment (start 143.860001 61.112998) (end 145.012974 59.960025) (width 0.45) (layer F.Cu) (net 4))
 (segment (start 146.622886 57.445001) (end 148.294999 57.445001) (width 0.45) (layer F.Cu) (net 6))
 (segment (start 143.060001 62.135) (end 143.060001 61.007886) (width 0.45) (layer F.Cu) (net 6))
 (segment (start 148.294999 57.445001) (end 149.86 55.88) (width 0.45) (layer F.Cu) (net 6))
 (segment (start 143.060001 61.007886) (end 146.622886 57.445001) (width 0.45) (layer F.Cu) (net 6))
 (segment (start 147.265001 55.88) (end 147.32 55.88) (width 0.45) (layer F.Cu) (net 7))
 (segment (start 142.260001 60.885) (end 147.265001 55.88) (width 0.45) (layer F.Cu) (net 7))
 (segment (start 142.260001 62.135) (end 142.260001 60.885) (width 0.45) (layer F.Cu) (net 7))
 (segment (start 158.44 66.04) (end 157.48 66.04) (width 0.45) (layer F.Cu) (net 10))
 (segment (start 159.3 71) (end 159.3 66.9) (width 0.45) (layer F.Cu) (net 10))
 (segment (start 157.2 73.1) (end 159.3 71) (width 0.45) (layer F.Cu) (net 10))
 (segment (start 145.075001 73.1) (end 157.2 73.1) (width 0.45) (layer F.Cu) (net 10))
 (segment (start 143.860001 71.885) (end 145.075001 73.1) (width 0.45) (layer F.Cu) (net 10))
 (segment (start 159.3 66.9) (end 158.44 66.04) (width 0.45) (layer F.Cu) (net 10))
 (segment (start 143.860001 70.635) (end 143.860001 71.885) (width 0.45) (layer F.Cu) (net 10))
 (segment (start 154.16 66.04) (end 154.94 66.04) (width 0.45) (layer F.Cu) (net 11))
 (segment (start 150.424999 69.775001) (end 154.16 66.04) (width 0.45) (layer F.Cu) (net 11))
 (segment (start 146.700002 69.775001) (end 150.424999 69.775001) (width 0.45) (layer F.Cu) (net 11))
 (segment (start 146.110001 69.185) (end 146.700002 69.775001) (width 0.45) (layer F.Cu) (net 11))
 (segment (start 152.98 68.58) (end 154.94 68.58) (width 0.45) (layer F.Cu) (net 12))
 (segment (start 150.924988 70.635012) (end 152.98 68.58) (width 0.45) (layer F.Cu) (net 12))
 (segment (start 150.185698 70.635012) (end 150.924988 70.635012) (width 0.45) (layer F.Cu) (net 12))
 (segment (start 150.185686 70.635) (end 150.185698 70.635012) (width 0.45) (layer F.Cu) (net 12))
 (segment (start 144.660001 70.635) (end 150.185686 70.635) (width 0.45) (layer F.Cu) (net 12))
 (segment (start 147.5 75.6) (end 153.7 75.6) (width 0.45) (layer F.Cu) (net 15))
 (segment (start 147.5 75.307998) (end 147.5 75.6) (width 0.45) (layer F.Cu) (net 15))
 (segment (start 146.492002 74.3) (end 147.5 75.307998) (width 0.45) (layer F.Cu) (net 15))
 (segment (start 143.875001 74.3) (end 146.492002 74.3) (width 0.45) (layer F.Cu) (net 15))
 (segment (start 141.460001 71.885) (end 143.875001 74.3) (width 0.45) (layer F.Cu) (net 15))
 (segment (start 141.460001 70.635) (end 141.460001 71.885) (width 0.45) (layer F.Cu) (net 15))
 (segment (start 135.78 73.915001) (end 139.060001 70.635) (width 0.45) (layer F.Cu) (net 13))
 (segment (start 135.78 75.64) (end 135.78 73.915001) (width 0.45) (layer F.Cu) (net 13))
 (segment (start 139.860001 74.099999) (end 139.860001 70.635) (width 0.45) (layer F.Cu) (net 14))
 (segment (start 138.32 75.64) (end 139.860001 74.099999) (width 0.45) (layer F.Cu) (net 14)))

